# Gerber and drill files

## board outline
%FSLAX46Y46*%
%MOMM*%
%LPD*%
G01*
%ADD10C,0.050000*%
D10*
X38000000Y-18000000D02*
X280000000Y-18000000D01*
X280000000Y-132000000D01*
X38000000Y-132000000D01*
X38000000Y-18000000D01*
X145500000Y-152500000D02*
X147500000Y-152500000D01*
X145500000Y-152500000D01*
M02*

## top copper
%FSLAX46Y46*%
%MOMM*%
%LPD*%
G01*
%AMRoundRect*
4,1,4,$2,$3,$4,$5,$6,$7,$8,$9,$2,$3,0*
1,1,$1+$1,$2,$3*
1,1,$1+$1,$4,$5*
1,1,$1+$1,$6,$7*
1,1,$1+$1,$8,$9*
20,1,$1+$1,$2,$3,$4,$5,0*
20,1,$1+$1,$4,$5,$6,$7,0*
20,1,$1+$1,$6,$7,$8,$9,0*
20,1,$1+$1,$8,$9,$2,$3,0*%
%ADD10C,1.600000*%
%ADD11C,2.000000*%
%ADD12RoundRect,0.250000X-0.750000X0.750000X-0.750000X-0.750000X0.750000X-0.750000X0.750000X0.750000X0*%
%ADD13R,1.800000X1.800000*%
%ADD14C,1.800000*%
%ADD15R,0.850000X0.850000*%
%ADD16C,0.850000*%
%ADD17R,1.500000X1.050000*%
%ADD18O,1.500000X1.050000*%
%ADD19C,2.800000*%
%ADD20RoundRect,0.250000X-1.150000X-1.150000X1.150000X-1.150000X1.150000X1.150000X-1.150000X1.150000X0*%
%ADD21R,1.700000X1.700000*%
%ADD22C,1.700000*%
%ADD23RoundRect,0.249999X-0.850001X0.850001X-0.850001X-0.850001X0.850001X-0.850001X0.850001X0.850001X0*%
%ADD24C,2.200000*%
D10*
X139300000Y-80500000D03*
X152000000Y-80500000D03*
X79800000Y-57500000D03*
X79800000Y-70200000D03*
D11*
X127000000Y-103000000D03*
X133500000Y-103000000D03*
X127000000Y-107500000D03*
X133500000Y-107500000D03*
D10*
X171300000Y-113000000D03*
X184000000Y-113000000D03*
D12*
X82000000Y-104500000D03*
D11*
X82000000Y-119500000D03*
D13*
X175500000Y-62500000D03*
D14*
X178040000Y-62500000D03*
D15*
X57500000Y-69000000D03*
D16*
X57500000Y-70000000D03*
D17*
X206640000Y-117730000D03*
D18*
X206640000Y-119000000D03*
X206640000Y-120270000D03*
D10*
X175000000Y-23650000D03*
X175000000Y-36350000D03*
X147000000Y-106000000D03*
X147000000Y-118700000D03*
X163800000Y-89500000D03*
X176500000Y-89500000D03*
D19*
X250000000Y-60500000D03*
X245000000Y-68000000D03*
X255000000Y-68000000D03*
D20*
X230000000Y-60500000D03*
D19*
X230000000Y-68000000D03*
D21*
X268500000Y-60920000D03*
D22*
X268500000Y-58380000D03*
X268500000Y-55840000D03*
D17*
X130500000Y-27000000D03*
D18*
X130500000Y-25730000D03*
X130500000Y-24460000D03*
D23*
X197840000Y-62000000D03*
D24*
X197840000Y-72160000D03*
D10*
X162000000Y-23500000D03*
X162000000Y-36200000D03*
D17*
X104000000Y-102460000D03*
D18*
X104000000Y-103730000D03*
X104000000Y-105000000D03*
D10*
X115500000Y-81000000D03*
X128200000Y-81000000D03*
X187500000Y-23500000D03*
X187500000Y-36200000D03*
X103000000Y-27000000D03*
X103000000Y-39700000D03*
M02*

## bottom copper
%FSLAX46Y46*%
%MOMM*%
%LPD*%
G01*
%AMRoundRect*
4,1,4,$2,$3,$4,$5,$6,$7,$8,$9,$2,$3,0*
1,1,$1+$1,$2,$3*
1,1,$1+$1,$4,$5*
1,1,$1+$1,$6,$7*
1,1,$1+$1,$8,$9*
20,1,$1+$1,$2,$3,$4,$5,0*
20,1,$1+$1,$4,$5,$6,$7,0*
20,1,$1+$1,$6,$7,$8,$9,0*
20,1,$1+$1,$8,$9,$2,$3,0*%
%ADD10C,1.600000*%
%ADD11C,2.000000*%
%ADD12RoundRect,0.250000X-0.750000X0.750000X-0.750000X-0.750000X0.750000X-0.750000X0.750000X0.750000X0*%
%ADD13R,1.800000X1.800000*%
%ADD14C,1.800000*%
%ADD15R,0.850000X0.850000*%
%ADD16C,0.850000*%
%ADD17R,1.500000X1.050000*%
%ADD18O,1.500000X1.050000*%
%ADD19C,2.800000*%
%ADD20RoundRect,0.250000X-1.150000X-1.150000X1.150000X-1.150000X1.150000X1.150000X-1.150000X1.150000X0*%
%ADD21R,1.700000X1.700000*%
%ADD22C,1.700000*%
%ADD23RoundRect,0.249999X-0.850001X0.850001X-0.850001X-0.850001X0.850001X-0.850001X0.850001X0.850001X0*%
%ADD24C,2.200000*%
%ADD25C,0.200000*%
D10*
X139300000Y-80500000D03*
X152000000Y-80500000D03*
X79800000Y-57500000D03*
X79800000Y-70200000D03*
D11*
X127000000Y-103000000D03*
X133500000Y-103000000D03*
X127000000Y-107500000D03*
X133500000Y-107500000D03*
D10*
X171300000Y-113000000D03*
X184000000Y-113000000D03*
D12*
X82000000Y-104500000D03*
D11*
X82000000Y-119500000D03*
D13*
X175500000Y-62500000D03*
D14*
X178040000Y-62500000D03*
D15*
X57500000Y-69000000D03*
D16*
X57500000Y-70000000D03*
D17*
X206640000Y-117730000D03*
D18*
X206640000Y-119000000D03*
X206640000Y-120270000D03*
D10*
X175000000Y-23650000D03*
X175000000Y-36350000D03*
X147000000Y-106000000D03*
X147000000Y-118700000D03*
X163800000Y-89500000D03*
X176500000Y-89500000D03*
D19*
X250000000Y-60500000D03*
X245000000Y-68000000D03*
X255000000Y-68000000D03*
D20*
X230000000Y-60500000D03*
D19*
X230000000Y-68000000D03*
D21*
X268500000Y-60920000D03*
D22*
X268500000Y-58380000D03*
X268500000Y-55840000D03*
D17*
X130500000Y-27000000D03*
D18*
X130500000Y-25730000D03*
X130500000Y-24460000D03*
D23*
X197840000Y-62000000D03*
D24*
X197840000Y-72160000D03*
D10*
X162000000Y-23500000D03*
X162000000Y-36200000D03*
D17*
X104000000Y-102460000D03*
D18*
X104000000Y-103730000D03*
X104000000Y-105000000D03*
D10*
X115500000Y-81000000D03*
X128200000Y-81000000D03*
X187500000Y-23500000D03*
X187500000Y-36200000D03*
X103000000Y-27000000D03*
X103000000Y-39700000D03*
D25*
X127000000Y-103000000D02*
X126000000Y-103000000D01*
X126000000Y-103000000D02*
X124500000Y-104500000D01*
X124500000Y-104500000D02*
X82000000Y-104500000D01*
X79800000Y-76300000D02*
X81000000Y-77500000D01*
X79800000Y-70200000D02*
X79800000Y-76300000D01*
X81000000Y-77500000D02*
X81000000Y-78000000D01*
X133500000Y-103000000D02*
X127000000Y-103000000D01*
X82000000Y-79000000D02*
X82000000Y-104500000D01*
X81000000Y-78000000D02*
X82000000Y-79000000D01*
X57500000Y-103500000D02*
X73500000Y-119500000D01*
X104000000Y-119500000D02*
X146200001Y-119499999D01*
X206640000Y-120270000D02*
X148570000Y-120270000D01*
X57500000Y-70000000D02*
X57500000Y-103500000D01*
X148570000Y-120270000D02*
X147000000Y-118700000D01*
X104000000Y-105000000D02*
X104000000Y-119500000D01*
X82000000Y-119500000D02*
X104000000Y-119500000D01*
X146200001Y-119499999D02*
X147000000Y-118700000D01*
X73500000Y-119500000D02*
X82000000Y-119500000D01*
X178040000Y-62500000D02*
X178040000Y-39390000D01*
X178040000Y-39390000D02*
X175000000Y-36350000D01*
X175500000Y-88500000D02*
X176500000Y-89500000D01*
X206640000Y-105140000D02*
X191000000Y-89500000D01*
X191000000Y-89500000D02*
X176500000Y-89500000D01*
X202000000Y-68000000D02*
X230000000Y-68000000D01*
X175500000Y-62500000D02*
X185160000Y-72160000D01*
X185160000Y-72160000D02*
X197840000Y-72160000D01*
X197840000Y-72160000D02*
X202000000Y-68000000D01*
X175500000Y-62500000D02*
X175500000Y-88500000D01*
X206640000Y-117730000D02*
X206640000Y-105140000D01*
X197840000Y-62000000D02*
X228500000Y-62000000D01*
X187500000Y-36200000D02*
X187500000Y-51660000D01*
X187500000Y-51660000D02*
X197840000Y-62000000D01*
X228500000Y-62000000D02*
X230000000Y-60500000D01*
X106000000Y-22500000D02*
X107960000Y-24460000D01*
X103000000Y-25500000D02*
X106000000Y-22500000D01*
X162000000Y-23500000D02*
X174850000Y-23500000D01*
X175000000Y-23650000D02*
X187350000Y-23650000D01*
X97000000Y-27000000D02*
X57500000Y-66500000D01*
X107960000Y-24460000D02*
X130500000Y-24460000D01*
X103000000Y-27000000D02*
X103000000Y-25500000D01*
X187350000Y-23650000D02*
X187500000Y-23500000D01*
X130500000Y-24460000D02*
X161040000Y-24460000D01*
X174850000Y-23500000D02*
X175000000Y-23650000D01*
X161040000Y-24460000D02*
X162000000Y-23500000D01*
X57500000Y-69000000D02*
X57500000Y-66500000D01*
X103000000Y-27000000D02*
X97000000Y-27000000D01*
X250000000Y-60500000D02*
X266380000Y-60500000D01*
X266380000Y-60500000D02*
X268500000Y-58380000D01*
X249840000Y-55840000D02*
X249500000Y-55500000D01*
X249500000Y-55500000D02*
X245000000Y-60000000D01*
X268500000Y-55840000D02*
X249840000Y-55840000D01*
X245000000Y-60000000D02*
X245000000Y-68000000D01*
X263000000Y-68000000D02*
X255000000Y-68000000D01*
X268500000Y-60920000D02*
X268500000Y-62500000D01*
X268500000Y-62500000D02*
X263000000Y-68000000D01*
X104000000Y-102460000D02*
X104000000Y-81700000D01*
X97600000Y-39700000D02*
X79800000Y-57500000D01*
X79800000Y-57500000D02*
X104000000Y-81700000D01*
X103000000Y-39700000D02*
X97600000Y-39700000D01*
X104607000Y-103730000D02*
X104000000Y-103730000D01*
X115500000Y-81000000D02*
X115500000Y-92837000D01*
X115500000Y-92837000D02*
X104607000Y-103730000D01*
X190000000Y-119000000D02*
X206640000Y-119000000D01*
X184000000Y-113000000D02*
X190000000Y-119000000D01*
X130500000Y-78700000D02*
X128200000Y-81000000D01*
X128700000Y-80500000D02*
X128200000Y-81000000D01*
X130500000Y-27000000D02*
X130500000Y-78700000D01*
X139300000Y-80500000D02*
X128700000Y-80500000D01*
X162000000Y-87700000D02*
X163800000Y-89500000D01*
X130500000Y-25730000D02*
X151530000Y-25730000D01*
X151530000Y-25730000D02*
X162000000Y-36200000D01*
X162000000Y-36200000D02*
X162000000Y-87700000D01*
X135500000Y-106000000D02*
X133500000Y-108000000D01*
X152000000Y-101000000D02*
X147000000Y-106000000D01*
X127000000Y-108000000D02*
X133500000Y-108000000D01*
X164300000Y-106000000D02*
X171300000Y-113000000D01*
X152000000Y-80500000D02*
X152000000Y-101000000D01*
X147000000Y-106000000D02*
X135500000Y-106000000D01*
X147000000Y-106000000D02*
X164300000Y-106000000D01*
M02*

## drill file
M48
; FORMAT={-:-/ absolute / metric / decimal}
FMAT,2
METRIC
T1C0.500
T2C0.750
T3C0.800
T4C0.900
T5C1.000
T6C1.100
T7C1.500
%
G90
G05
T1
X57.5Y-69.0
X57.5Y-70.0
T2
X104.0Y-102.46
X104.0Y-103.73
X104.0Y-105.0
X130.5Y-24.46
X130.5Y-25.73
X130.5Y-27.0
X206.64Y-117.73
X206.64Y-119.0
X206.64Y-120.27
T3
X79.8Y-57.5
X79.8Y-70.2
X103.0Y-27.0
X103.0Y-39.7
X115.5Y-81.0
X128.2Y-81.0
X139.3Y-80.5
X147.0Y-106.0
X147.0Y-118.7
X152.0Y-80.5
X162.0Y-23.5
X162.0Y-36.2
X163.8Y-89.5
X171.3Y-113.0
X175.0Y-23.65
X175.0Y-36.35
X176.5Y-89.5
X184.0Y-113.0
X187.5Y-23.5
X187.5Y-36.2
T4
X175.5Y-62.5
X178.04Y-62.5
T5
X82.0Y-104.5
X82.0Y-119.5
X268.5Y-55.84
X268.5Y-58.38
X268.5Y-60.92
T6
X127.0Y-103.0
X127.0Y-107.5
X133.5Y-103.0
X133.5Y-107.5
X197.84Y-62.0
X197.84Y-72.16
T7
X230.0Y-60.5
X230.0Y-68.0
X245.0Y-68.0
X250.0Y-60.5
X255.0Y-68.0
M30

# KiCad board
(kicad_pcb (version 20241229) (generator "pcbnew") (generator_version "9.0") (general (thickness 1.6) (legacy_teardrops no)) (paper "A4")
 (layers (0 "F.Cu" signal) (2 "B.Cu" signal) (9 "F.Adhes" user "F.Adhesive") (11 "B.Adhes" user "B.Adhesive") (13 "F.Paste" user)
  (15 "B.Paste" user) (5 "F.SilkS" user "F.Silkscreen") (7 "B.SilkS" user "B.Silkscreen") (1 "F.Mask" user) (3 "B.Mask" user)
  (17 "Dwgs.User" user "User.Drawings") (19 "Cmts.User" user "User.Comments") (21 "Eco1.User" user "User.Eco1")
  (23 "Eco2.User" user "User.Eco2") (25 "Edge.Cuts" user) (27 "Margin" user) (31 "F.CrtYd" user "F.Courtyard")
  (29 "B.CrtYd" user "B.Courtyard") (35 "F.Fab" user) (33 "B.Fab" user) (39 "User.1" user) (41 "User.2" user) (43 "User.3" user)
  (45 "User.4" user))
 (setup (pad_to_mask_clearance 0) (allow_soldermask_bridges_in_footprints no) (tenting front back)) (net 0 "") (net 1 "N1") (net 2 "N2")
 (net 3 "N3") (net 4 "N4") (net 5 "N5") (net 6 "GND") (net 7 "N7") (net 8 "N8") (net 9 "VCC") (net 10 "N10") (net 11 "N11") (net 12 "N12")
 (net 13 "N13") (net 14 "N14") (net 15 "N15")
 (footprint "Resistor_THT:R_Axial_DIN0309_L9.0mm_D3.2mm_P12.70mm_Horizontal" (layer "F.Cu") (at 139.3 80.5)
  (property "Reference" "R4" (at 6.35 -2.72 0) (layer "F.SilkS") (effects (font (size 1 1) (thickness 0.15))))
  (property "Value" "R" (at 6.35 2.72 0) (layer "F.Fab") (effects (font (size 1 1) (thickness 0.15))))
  (pad "1" thru_hole circle (at 0 0) (size 1.6 1.6) (drill 0.8) (layers "*.Cu" "*.Mask") (remove_unused_layers no) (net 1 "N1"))
  (pad "2" thru_hole circle (at 12.7 0) (size 1.6 1.6) (drill 0.8) (layers "*.Cu" "*.Mask") (remove_unused_layers no) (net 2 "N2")))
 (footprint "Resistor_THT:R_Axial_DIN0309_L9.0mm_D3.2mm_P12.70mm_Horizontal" (layer "F.Cu") (at 79.8 57.5 -90)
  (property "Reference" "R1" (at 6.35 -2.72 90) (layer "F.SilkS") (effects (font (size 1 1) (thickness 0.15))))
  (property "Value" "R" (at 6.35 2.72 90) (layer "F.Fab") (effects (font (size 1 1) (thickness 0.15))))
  (pad "1" thru_hole circle (at 0 0 270) (size 1.6 1.6) (drill 0.8) (layers "*.Cu" "*.Mask") (remove_unused_layers no) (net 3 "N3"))
  (pad "2" thru_hole circle (at 12.7 0 270) (size 1.6 1.6) (drill 0.8) (layers "*.Cu" "*.Mask") (remove_unused_layers no) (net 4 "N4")))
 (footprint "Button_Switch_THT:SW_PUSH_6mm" (layer "F.Cu") (at 127 103)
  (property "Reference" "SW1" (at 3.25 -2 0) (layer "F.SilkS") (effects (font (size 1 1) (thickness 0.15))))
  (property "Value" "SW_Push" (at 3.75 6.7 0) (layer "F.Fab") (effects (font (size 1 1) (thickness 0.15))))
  (pad "1" thru_hole circle (at 0 0 90) (size 2 2) (drill 1.1) (layers "*.Cu" "*.Mask") (remove_unused_layers no) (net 4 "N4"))
  (pad "1" thru_hole circle (at 6.5 0 90) (size 2 2) (drill 1.1) (layers "*.Cu" "*.Mask") (remove_unused_layers no) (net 4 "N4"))
  (pad "2" thru_hole circle (at 0 4.5 90) (size 2 2) (drill 1.1) (layers "*.Cu" "*.Mask") (remove_unused_layers no) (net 2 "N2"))
  (pad "2" thru_hole circle (at 6.5 4.5 90) (size 2 2) (drill 1.1) (layers "*.Cu" "*.Mask") (remove_unused_layers no) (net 2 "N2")))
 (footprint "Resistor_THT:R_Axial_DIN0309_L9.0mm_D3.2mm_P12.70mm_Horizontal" (layer "F.Cu") (at 171.3 113)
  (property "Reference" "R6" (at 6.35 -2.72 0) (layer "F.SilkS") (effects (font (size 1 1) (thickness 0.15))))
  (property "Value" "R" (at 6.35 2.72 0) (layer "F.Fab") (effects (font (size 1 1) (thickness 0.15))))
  (pad "1" thru_hole circle (at 0 0) (size 1.6 1.6) (drill 0.8) (layers "*.Cu" "*.Mask") (remove_unused_layers no) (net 2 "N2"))
  (pad "2" thru_hole circle (at 12.7 0) (size 1.6 1.6) (drill 0.8) (layers "*.Cu" "*.Mask") (remove_unused_layers no) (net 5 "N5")))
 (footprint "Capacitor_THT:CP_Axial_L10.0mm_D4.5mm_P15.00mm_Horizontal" (layer "F.Cu") (at 82 104.5 -90)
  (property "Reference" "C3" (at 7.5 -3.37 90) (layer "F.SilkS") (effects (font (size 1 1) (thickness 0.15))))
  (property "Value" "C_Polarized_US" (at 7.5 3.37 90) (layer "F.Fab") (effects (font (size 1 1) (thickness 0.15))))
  (pad "1" thru_hole roundrect (at 0 0 270) (size 2 2) (drill 1) (layers "*.Cu" "*.Mask") (remove_unused_layers no) (roundrect_rratio 0.125)
   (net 4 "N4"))
  (pad "2" thru_hole circle (at 15 0 270) (size 2 2) (drill 1) (layers "*.Cu" "*.Mask") (remove_unused_layers no) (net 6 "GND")))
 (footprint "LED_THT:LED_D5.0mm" (layer "F.Cu") (at 175.5 62.5)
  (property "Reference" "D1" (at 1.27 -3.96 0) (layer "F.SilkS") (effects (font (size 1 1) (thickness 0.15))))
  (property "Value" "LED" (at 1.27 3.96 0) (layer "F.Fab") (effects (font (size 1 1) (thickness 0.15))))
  (pad "1" thru_hole rect (at 0 0) (size 1.8 1.8) (drill 0.9) (layers "*.Cu" "*.Mask") (remove_unused_layers no) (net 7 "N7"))
  (pad "2" thru_hole circle (at 2.54 0) (size 1.8 1.8) (drill 0.9) (layers "*.Cu" "*.Mask") (remove_unused_layers no) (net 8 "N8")))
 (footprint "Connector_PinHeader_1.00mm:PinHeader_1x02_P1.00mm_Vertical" (layer "F.Cu") (at 57.5 69)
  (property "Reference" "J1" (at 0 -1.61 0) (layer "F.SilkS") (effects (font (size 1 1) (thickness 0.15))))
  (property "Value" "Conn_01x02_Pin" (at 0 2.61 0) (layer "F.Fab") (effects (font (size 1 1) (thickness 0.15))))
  (pad "1" thru_hole rect (at 0 0) (size 0.85 0.85) (drill 0.5) (layers "*.Cu" "*.Mask") (remove_unused_layers no) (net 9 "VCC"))
  (pad "2" thru_hole circle (at 0 1) (size 0.85 0.85) (drill 0.5) (layers "*.Cu" "*.Mask") (remove_unused_layers no) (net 6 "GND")))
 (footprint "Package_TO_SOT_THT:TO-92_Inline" (layer "F.Cu") (at 206.64 117.73 -90)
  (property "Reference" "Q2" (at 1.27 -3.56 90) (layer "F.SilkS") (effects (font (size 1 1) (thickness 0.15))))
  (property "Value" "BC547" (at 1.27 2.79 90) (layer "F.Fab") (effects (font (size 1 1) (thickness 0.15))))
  (pad "1" thru_hole rect (at 0 0 270) (size 1.05 1.5) (drill 0.75) (layers "*.Cu" "*.Mask") (remove_unused_layers no) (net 7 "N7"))
  (pad "2" thru_hole oval (at 1.27 0 270) (size 1.05 1.5) (drill 0.75) (layers "*.Cu" "*.Mask") (remove_unused_layers no) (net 5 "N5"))
  (pad "3" thru_hole oval (at 2.54 0 270) (size 1.05 1.5) (drill 0.75) (layers "*.Cu" "*.Mask") (remove_unused_layers no) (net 6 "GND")))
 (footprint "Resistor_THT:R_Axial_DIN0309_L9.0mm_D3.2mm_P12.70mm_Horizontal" (layer "F.Cu") (at 175 23.65 -90)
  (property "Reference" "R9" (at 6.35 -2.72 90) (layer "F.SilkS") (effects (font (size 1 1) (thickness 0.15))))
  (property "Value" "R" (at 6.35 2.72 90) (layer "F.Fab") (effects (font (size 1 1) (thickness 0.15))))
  (pad "1" thru_hole circle (at 0 0 270) (size 1.6 1.6) (drill 0.8) (layers "*.Cu" "*.Mask") (remove_unused_layers no) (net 9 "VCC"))
  (pad "2" thru_hole circle (at 12.7 0 270) (size 1.6 1.6) (drill 0.8) (layers "*.Cu" "*.Mask") (remove_unused_layers no) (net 8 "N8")))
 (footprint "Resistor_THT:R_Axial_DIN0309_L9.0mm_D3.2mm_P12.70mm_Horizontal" (layer "F.Cu") (at 147 106 -90)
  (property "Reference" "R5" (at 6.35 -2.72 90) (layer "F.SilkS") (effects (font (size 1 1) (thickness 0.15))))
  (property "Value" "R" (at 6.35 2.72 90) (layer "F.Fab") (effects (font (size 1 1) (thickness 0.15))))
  (pad "1" thru_hole circle (at 0 0 270) (size 1.6 1.6) (drill 0.8) (layers "*.Cu" "*.Mask") (remove_unused_layers no) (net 2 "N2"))
  (pad "2" thru_hole circle (at 12.7 0 270) (size 1.6 1.6) (drill 0.8) (layers "*.Cu" "*.Mask") (remove_unused_layers no) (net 6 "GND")))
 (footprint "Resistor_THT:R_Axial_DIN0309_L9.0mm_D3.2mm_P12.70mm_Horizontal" (layer "F.Cu") (at 163.8 89.5)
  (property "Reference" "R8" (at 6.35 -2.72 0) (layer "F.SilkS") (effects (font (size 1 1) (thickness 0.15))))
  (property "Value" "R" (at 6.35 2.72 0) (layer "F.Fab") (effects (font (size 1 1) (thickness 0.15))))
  (pad "1" thru_hole circle (at 0 0) (size 1.6 1.6) (drill 0.8) (layers "*.Cu" "*.Mask") (remove_unused_layers no) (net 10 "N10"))
  (pad "2" thru_hole circle (at 12.7 0) (size 1.6 1.6) (drill 0.8) (layers "*.Cu" "*.Mask") (remove_unused_layers no) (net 7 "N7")))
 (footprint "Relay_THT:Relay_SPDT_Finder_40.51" (layer "F.Cu") (at 230 60.5)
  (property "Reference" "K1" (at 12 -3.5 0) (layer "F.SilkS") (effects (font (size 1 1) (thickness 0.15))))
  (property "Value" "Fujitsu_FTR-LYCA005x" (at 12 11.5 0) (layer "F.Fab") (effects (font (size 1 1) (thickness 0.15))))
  (pad "11" thru_hole circle (at 20 0) (size 2.8 2.8) (drill 1.5) (layers "*.Cu" "*.Mask") (remove_unused_layers no) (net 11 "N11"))
  (pad "12" thru_hole circle (at 15 7.5) (size 2.8 2.8) (drill 1.5) (layers "*.Cu" "*.Mask") (remove_unused_layers no) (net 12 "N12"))
  (pad "14" thru_hole circle (at 25 7.5) (size 2.8 2.8) (drill 1.5) (layers "*.Cu" "*.Mask") (remove_unused_layers no) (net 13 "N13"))
  (pad "A1" thru_hole roundrect (at 0 0) (size 2.8 2.8) (drill 1.5) (layers "*.Cu" "*.Mask") (remove_unused_layers no)
   (roundrect_rratio 0.08928571429) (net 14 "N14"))
  (pad "A2" thru_hole circle (at 0 7.5) (size 2.8 2.8) (drill 1.5) (layers "*.Cu" "*.Mask") (remove_unused_layers no) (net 7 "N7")))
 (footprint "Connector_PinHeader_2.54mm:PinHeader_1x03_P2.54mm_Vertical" (layer "F.Cu") (at 268.5 60.92 180)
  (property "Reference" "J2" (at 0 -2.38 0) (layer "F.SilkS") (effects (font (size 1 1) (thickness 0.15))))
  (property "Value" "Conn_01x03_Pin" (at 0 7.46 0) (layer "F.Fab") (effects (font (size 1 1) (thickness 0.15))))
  (pad "1" thru_hole rect (at 0 0 180) (size 1.7 1.7) (drill 1) (layers "*.Cu" "*.Mask") (remove_unused_layers no) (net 13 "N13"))
  (pad "2" thru_hole circle (at 0 2.54 180) (size 1.7 1.7) (drill 1) (layers "*.Cu" "*.Mask") (remove_unused_layers no) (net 11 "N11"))
  (pad "3" thru_hole circle (at 0 5.08 180) (size 1.7 1.7) (drill 1) (layers "*.Cu" "*.Mask") (remove_unused_layers no) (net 12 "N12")))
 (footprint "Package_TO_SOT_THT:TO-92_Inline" (layer "F.Cu") (at 130.5 27 90)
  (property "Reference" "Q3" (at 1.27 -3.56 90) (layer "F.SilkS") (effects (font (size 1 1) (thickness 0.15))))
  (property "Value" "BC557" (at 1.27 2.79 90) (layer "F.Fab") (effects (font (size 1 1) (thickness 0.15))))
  (pad "1" thru_hole rect (at 0 0 90) (size 1.05 1.5) (drill 0.75) (layers "*.Cu" "*.Mask") (remove_unused_layers no) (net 1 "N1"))
  (pad "2" thru_hole oval (at 1.27 0 90) (size 1.05 1.5) (drill 0.75) (layers "*.Cu" "*.Mask") (remove_unused_layers no) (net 10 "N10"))
  (pad "3" thru_hole oval (at 2.54 0 90) (size 1.05 1.5) (drill 0.75) (layers "*.Cu" "*.Mask") (remove_unused_layers no) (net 9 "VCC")))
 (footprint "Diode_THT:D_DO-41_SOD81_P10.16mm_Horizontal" (layer "F.Cu") (at 197.84 62 -90)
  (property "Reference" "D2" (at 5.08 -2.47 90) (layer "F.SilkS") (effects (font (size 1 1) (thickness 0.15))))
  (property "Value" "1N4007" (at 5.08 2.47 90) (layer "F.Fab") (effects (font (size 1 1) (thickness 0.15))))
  (pad "1" thru_hole roundrect (at 0 0 270) (size 2.2 2.2) (drill 1.1) (layers "*.Cu" "*.Mask") (remove_unused_layers no)
   (roundrect_rratio 0.113636) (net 14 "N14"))
  (pad "2" thru_hole circle (at 10.16 0 270) (size 2.2 2.2) (drill 1.1) (layers "*.Cu" "*.Mask") (remove_unused_layers no) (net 7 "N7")))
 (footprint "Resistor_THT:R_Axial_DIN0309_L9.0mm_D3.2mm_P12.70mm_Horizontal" (layer "F.Cu") (at 162 23.5 -90)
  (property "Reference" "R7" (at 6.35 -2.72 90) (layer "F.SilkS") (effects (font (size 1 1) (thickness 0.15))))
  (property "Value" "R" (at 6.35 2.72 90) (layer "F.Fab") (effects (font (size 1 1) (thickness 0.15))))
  (pad "1" thru_hole circle (at 0 0 270) (size 1.6 1.6) (drill 0.8) (layers "*.Cu" "*.Mask") (remove_unused_layers no) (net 9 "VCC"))
  (pad "2" thru_hole circle (at 12.7 0 270) (size 1.6 1.6) (drill 0.8) (layers "*.Cu" "*.Mask") (remove_unused_layers no) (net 10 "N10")))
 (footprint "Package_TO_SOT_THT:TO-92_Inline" (layer "F.Cu") (at 104 102.46 -90)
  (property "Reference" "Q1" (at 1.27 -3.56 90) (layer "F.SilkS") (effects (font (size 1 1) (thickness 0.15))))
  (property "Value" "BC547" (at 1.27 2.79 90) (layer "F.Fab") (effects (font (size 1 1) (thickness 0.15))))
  (pad "1" thru_hole rect (at 0 0 270) (size 1.05 1.5) (drill 0.75) (layers "*.Cu" "*.Mask") (remove_unused_layers no) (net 3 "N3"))
  (pad "2" thru_hole oval (at 1.27 0 270) (size 1.05 1.5) (drill 0.75) (layers "*.Cu" "*.Mask") (remove_unused_layers no) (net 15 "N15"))
  (pad "3" thru_hole oval (at 2.54 0 270) (size 1.05 1.5) (drill 0.75) (layers "*.Cu" "*.Mask") (remove_unused_layers no) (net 6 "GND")))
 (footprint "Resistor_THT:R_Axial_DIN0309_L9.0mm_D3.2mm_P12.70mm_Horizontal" (layer "F.Cu") (at 115.5 81)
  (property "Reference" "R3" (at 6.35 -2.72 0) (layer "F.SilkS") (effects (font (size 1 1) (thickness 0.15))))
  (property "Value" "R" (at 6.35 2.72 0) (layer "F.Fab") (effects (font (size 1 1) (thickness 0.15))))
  (pad "1" thru_hole circle (at 0 0) (size 1.6 1.6) (drill 0.8) (layers "*.Cu" "*.Mask") (remove_unused_layers no) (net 15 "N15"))
  (pad "2" thru_hole circle (at 12.7 0) (size 1.6 1.6) (drill 0.8) (layers "*.Cu" "*.Mask") (remove_unused_layers no) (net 1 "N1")))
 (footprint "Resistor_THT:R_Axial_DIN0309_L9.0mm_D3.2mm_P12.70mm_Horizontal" (layer "F.Cu") (at 187.5 23.5 -90)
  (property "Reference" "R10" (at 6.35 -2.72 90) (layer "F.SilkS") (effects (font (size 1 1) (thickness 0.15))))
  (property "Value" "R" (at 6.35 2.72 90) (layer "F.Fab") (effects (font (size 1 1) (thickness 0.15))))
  (pad "1" thru_hole circle (at 0 0 270) (size 1.6 1.6) (drill 0.8) (layers "*.Cu" "*.Mask") (remove_unused_layers no) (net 9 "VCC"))
  (pad "2" thru_hole circle (at 12.7 0 270) (size 1.6 1.6) (drill 0.8) (layers "*.Cu" "*.Mask") (remove_unused_layers no) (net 14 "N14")))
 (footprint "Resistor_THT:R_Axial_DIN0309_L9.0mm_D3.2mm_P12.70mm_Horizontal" (layer "F.Cu") (at 103 27 -90)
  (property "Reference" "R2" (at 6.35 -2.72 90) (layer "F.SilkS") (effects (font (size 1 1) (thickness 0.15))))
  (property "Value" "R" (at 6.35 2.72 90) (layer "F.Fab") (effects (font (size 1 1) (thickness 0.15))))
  (pad "1" thru_hole circle (at 0 0 270) (size 1.6 1.6) (drill 0.8) (layers "*.Cu" "*.Mask") (remove_unused_layers no) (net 9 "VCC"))
  (pad "2" thru_hole circle (at 12.7 0 270) (size 1.6 1.6) (drill 0.8) (layers "*.Cu" "*.Mask") (remove_unused_layers no) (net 3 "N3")))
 (gr_rect (start 38 18) (end 280 132) (stroke (width 0.05) (type default)) (fill no) (layer "Edge.Cuts"))
 (gr_rect (start 145.5 152.5) (end 147.5 152.5) (stroke (width 0.05) (type default)) (fill no) (layer "Edge.Cuts"))
 (segment (start 127 103) (end 126 103) (width 0.2) (layer "B.Cu") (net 4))
 (segment (start 126 103) (end 124.5 104.5) (width 0.2) (layer "B.Cu") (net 4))
 (segment (start 124.5 104.5) (end 82 104.5) (width 0.2) (layer "B.Cu") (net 4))
 (segment (start 79.8 76.3) (end 81 77.5) (width 0.2) (layer "B.Cu") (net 4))
 (segment (start 79.8 70.2) (end 79.8 76.3) (width 0.2) (layer "B.Cu") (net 4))
 (segment (start 81 77.5) (end 81 78) (width 0.2) (layer "B.Cu") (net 4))
 (segment (start 133.5 103) (end 127 103) (width 0.2) (layer "B.Cu") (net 4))
 (segment (start 82 79) (end 82 104.5) (width 0.2) (layer "B.Cu") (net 4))
 (segment (start 81 78) (end 82 79) (width 0.2) (layer "B.Cu") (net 4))
 (segment (start 57.5 103.5) (end 73.5 119.5) (width 0.2) (layer "B.Cu") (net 6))
 (segment (start 104 119.5) (end 146.200001 119.499999) (width 0.2) (layer "B.Cu") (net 6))
 (segment (start 206.64 120.27) (end 148.57 120.27) (width 0.2) (layer "B.Cu") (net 6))
 (segment (start 57.5 70) (end 57.5 103.5) (width 0.2) (layer "B.Cu") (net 6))
 (segment (start 148.57 120.27) (end 147 118.7) (width 0.2) (layer "B.Cu") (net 6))
 (segment (start 104 105) (end 104 119.5) (width 0.2) (layer "B.Cu") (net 6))
 (segment (start 82 119.5) (end 104 119.5) (width 0.2) (layer "B.Cu") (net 6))
 (segment (start 146.200001 119.499999) (end 147 118.7) (width 0.2) (layer "B.Cu") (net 6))
 (segment (start 73.5 119.5) (end 82 119.5) (width 0.2) (layer "B.Cu") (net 6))
 (segment (start 178.04 62.5) (end 178.04 39.39) (width 0.2) (layer "B.Cu") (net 8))
 (segment (start 178.04 39.39) (end 175 36.35) (width 0.2) (layer "B.Cu") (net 8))
 (segment (start 175.5 88.5) (end 176.5 89.5) (width 0.2) (layer "B.Cu") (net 7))
 (segment (start 206.64 105.14) (end 191 89.5) (width 0.2) (layer "B.Cu") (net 7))
 (segment (start 191 89.5) (end 176.5 89.5) (width 0.2) (layer "B.Cu") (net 7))
 (segment (start 202 68) (end 230 68) (width 0.2) (layer "B.Cu") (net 7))
 (segment (start 175.5 62.5) (end 185.16 72.16) (width 0.2) (layer "B.Cu") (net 7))
 (segment (start 185.16 72.16) (end 197.84 72.16) (width 0.2) (layer "B.Cu") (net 7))
 (segment (start 197.84 72.16) (end 202 68) (width 0.2) (layer "B.Cu") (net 7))
 (segment (start 175.5 62.5) (end 175.5 88.5) (width 0.2) (layer "B.Cu") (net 7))
 (segment (start 206.64 117.73) (end 206.64 105.14) (width 0.2) (layer "B.Cu") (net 7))
 (segment (start 197.84 62) (end 228.5 62) (width 0.2) (layer "B.Cu") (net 14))
 (segment (start 187.5 36.2) (end 187.5 51.66) (width 0.2) (layer "B.Cu") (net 14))
 (segment (start 187.5 51.66) (end 197.84 62) (width 0.2) (layer "B.Cu") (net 14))
 (segment (start 228.5 62) (end 230 60.5) (width 0.2) (layer "B.Cu") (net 14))
 (segment (start 106 22.5) (end 107.96 24.46) (width 0.2) (layer "B.Cu") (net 9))
 (segment (start 103 25.5) (end 106 22.5) (width 0.2) (layer "B.Cu") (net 9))
 (segment (start 162 23.5) (end 174.85 23.5) (width 0.2) (layer "B.Cu") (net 9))
 (segment (start 175 23.65) (end 187.35 23.65) (width 0.2) (layer "B.Cu") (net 9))
 (segment (start 97 27) (end 57.5 66.5) (width 0.2) (layer "B.Cu") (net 9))
 (segment (start 107.96 24.46) (end 130.5 24.46) (width 0.2) (layer "B.Cu") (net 9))
 (segment (start 103 27) (end 103 25.5) (width 0.2) (layer "B.Cu") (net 9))
 (segment (start 187.35 23.65) (end 187.5 23.5) (width 0.2) (layer "B.Cu") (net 9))
 (segment (start 130.5 24.46) (end 161.04 24.46) (width 0.2) (layer "B.Cu") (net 9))
 (segment (start 174.85 23.5) (end 175 23.65) (width 0.2) (layer "B.Cu") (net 9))
 (segment (start 161.04 24.46) (end 162 23.5) (width 0.2) (layer "B.Cu") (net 9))
 (segment (start 57.5 69) (end 57.5 66.5) (width 0.2) (layer "B.Cu") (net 9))
 (segment (start 103 27) (end 97 27) (width 0.2) (layer "B.Cu") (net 9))
 (segment (start 250 60.5) (end 266.38 60.5) (width 0.2) (layer "B.Cu") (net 11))
 (segment (start 266.38 60.5) (end 268.5 58.38) (width 0.2) (layer "B.Cu") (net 11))
 (segment (start 249.84 55.84) (end 249.5 55.5) (width 0.2) (layer "B.Cu") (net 12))
 (segment (start 249.5 55.5) (end 245 60) (width 0.2) (layer "B.Cu") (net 12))
 (segment (start 268.5 55.84) (end 249.84 55.84) (width 0.2) (layer "B.Cu") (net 12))
 (segment (start 245 60) (end 245 68) (width 0.2) (layer "B.Cu") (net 12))
 (segment (start 263 68) (end 255 68) (width 0.2) (layer "B.Cu") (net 13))
 (segment (start 268.5 60.92) (end 268.5 62.5) (width 0.2) (layer "B.Cu") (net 13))
 (segment (start 268.5 62.5) (end 263 68) (width 0.2) (layer "B.Cu") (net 13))
 (segment (start 104 102.46) (end 104 81.7) (width 0.2) (layer "B.Cu") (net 3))
 (segment (start 97.6 39.7) (end 79.8 57.5) (width 0.2) (layer "B.Cu") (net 3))
 (segment (start 79.8 57.5) (end 104 81.7) (width 0.2) (layer "B.Cu") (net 3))
 (segment (start 103 39.7) (end 97.6 39.7) (width 0.2) (layer "B.Cu") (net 3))
 (segment (start 104.607 103.73) (end 104 103.73) (width 0.2) (layer "B.Cu") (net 15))
 (segment (start 115.5 81) (end 115.5 92.837) (width 0.2) (layer "B.Cu") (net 15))
 (segment (start 115.5 92.837) (end 104.607 103.73) (width 0.2) (layer "B.Cu") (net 15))
 (segment (start 190 119) (end 206.64 119) (width 0.2) (layer "B.Cu") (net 5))
 (segment (start 184 113) (end 190 119) (width 0.2) (layer "B.Cu") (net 5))
 (segment (start 130.5 78.7) (end 128.2 81) (width 0.2) (layer "B.Cu") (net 1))
 (segment (start 128.7 80.5) (end 128.2 81) (width 0.2) (layer "B.Cu") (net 1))
 (segment (start 130.5 27) (end 130.5 78.7) (width 0.2) (layer "B.Cu") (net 1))
 (segment (start 139.3 80.5) (end 128.7 80.5) (width 0.2) (layer "B.Cu") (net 1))
 (segment (start 162 87.7) (end 163.8 89.5) (width 0.2) (layer "B.Cu") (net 10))
 (segment (start 130.5 25.73) (end 151.53 25.73) (width 0.2) (layer "B.Cu") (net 10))
 (segment (start 151.53 25.73) (end 162 36.2) (width 0.2) (layer "B.Cu") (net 10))
 (segment (start 162 36.2) (end 162 87.7) (width 0.2) (layer "B.Cu") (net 10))
 (segment (start 135.5 106) (end 133.5 108) (width 0.2) (layer "B.Cu") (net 2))
 (segment (start 152 101) (end 147 106) (width 0.2) (layer "B.Cu") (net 2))
 (segment (start 127 108) (end 133.5 108) (width 0.2) (layer "B.Cu") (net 2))
 (segment (start 164.3 106) (end 171.3 113) (width 0.2) (layer "B.Cu") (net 2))
 (segment (start 152 80.5) (end 152 101) (width 0.2) (layer "B.Cu") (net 2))
 (segment (start 147 106) (end 135.5 106) (width 0.2) (layer "B.Cu") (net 2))
 (segment (start 147 106) (end 164.3 106) (width 0.2) (layer "B.Cu") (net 2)))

